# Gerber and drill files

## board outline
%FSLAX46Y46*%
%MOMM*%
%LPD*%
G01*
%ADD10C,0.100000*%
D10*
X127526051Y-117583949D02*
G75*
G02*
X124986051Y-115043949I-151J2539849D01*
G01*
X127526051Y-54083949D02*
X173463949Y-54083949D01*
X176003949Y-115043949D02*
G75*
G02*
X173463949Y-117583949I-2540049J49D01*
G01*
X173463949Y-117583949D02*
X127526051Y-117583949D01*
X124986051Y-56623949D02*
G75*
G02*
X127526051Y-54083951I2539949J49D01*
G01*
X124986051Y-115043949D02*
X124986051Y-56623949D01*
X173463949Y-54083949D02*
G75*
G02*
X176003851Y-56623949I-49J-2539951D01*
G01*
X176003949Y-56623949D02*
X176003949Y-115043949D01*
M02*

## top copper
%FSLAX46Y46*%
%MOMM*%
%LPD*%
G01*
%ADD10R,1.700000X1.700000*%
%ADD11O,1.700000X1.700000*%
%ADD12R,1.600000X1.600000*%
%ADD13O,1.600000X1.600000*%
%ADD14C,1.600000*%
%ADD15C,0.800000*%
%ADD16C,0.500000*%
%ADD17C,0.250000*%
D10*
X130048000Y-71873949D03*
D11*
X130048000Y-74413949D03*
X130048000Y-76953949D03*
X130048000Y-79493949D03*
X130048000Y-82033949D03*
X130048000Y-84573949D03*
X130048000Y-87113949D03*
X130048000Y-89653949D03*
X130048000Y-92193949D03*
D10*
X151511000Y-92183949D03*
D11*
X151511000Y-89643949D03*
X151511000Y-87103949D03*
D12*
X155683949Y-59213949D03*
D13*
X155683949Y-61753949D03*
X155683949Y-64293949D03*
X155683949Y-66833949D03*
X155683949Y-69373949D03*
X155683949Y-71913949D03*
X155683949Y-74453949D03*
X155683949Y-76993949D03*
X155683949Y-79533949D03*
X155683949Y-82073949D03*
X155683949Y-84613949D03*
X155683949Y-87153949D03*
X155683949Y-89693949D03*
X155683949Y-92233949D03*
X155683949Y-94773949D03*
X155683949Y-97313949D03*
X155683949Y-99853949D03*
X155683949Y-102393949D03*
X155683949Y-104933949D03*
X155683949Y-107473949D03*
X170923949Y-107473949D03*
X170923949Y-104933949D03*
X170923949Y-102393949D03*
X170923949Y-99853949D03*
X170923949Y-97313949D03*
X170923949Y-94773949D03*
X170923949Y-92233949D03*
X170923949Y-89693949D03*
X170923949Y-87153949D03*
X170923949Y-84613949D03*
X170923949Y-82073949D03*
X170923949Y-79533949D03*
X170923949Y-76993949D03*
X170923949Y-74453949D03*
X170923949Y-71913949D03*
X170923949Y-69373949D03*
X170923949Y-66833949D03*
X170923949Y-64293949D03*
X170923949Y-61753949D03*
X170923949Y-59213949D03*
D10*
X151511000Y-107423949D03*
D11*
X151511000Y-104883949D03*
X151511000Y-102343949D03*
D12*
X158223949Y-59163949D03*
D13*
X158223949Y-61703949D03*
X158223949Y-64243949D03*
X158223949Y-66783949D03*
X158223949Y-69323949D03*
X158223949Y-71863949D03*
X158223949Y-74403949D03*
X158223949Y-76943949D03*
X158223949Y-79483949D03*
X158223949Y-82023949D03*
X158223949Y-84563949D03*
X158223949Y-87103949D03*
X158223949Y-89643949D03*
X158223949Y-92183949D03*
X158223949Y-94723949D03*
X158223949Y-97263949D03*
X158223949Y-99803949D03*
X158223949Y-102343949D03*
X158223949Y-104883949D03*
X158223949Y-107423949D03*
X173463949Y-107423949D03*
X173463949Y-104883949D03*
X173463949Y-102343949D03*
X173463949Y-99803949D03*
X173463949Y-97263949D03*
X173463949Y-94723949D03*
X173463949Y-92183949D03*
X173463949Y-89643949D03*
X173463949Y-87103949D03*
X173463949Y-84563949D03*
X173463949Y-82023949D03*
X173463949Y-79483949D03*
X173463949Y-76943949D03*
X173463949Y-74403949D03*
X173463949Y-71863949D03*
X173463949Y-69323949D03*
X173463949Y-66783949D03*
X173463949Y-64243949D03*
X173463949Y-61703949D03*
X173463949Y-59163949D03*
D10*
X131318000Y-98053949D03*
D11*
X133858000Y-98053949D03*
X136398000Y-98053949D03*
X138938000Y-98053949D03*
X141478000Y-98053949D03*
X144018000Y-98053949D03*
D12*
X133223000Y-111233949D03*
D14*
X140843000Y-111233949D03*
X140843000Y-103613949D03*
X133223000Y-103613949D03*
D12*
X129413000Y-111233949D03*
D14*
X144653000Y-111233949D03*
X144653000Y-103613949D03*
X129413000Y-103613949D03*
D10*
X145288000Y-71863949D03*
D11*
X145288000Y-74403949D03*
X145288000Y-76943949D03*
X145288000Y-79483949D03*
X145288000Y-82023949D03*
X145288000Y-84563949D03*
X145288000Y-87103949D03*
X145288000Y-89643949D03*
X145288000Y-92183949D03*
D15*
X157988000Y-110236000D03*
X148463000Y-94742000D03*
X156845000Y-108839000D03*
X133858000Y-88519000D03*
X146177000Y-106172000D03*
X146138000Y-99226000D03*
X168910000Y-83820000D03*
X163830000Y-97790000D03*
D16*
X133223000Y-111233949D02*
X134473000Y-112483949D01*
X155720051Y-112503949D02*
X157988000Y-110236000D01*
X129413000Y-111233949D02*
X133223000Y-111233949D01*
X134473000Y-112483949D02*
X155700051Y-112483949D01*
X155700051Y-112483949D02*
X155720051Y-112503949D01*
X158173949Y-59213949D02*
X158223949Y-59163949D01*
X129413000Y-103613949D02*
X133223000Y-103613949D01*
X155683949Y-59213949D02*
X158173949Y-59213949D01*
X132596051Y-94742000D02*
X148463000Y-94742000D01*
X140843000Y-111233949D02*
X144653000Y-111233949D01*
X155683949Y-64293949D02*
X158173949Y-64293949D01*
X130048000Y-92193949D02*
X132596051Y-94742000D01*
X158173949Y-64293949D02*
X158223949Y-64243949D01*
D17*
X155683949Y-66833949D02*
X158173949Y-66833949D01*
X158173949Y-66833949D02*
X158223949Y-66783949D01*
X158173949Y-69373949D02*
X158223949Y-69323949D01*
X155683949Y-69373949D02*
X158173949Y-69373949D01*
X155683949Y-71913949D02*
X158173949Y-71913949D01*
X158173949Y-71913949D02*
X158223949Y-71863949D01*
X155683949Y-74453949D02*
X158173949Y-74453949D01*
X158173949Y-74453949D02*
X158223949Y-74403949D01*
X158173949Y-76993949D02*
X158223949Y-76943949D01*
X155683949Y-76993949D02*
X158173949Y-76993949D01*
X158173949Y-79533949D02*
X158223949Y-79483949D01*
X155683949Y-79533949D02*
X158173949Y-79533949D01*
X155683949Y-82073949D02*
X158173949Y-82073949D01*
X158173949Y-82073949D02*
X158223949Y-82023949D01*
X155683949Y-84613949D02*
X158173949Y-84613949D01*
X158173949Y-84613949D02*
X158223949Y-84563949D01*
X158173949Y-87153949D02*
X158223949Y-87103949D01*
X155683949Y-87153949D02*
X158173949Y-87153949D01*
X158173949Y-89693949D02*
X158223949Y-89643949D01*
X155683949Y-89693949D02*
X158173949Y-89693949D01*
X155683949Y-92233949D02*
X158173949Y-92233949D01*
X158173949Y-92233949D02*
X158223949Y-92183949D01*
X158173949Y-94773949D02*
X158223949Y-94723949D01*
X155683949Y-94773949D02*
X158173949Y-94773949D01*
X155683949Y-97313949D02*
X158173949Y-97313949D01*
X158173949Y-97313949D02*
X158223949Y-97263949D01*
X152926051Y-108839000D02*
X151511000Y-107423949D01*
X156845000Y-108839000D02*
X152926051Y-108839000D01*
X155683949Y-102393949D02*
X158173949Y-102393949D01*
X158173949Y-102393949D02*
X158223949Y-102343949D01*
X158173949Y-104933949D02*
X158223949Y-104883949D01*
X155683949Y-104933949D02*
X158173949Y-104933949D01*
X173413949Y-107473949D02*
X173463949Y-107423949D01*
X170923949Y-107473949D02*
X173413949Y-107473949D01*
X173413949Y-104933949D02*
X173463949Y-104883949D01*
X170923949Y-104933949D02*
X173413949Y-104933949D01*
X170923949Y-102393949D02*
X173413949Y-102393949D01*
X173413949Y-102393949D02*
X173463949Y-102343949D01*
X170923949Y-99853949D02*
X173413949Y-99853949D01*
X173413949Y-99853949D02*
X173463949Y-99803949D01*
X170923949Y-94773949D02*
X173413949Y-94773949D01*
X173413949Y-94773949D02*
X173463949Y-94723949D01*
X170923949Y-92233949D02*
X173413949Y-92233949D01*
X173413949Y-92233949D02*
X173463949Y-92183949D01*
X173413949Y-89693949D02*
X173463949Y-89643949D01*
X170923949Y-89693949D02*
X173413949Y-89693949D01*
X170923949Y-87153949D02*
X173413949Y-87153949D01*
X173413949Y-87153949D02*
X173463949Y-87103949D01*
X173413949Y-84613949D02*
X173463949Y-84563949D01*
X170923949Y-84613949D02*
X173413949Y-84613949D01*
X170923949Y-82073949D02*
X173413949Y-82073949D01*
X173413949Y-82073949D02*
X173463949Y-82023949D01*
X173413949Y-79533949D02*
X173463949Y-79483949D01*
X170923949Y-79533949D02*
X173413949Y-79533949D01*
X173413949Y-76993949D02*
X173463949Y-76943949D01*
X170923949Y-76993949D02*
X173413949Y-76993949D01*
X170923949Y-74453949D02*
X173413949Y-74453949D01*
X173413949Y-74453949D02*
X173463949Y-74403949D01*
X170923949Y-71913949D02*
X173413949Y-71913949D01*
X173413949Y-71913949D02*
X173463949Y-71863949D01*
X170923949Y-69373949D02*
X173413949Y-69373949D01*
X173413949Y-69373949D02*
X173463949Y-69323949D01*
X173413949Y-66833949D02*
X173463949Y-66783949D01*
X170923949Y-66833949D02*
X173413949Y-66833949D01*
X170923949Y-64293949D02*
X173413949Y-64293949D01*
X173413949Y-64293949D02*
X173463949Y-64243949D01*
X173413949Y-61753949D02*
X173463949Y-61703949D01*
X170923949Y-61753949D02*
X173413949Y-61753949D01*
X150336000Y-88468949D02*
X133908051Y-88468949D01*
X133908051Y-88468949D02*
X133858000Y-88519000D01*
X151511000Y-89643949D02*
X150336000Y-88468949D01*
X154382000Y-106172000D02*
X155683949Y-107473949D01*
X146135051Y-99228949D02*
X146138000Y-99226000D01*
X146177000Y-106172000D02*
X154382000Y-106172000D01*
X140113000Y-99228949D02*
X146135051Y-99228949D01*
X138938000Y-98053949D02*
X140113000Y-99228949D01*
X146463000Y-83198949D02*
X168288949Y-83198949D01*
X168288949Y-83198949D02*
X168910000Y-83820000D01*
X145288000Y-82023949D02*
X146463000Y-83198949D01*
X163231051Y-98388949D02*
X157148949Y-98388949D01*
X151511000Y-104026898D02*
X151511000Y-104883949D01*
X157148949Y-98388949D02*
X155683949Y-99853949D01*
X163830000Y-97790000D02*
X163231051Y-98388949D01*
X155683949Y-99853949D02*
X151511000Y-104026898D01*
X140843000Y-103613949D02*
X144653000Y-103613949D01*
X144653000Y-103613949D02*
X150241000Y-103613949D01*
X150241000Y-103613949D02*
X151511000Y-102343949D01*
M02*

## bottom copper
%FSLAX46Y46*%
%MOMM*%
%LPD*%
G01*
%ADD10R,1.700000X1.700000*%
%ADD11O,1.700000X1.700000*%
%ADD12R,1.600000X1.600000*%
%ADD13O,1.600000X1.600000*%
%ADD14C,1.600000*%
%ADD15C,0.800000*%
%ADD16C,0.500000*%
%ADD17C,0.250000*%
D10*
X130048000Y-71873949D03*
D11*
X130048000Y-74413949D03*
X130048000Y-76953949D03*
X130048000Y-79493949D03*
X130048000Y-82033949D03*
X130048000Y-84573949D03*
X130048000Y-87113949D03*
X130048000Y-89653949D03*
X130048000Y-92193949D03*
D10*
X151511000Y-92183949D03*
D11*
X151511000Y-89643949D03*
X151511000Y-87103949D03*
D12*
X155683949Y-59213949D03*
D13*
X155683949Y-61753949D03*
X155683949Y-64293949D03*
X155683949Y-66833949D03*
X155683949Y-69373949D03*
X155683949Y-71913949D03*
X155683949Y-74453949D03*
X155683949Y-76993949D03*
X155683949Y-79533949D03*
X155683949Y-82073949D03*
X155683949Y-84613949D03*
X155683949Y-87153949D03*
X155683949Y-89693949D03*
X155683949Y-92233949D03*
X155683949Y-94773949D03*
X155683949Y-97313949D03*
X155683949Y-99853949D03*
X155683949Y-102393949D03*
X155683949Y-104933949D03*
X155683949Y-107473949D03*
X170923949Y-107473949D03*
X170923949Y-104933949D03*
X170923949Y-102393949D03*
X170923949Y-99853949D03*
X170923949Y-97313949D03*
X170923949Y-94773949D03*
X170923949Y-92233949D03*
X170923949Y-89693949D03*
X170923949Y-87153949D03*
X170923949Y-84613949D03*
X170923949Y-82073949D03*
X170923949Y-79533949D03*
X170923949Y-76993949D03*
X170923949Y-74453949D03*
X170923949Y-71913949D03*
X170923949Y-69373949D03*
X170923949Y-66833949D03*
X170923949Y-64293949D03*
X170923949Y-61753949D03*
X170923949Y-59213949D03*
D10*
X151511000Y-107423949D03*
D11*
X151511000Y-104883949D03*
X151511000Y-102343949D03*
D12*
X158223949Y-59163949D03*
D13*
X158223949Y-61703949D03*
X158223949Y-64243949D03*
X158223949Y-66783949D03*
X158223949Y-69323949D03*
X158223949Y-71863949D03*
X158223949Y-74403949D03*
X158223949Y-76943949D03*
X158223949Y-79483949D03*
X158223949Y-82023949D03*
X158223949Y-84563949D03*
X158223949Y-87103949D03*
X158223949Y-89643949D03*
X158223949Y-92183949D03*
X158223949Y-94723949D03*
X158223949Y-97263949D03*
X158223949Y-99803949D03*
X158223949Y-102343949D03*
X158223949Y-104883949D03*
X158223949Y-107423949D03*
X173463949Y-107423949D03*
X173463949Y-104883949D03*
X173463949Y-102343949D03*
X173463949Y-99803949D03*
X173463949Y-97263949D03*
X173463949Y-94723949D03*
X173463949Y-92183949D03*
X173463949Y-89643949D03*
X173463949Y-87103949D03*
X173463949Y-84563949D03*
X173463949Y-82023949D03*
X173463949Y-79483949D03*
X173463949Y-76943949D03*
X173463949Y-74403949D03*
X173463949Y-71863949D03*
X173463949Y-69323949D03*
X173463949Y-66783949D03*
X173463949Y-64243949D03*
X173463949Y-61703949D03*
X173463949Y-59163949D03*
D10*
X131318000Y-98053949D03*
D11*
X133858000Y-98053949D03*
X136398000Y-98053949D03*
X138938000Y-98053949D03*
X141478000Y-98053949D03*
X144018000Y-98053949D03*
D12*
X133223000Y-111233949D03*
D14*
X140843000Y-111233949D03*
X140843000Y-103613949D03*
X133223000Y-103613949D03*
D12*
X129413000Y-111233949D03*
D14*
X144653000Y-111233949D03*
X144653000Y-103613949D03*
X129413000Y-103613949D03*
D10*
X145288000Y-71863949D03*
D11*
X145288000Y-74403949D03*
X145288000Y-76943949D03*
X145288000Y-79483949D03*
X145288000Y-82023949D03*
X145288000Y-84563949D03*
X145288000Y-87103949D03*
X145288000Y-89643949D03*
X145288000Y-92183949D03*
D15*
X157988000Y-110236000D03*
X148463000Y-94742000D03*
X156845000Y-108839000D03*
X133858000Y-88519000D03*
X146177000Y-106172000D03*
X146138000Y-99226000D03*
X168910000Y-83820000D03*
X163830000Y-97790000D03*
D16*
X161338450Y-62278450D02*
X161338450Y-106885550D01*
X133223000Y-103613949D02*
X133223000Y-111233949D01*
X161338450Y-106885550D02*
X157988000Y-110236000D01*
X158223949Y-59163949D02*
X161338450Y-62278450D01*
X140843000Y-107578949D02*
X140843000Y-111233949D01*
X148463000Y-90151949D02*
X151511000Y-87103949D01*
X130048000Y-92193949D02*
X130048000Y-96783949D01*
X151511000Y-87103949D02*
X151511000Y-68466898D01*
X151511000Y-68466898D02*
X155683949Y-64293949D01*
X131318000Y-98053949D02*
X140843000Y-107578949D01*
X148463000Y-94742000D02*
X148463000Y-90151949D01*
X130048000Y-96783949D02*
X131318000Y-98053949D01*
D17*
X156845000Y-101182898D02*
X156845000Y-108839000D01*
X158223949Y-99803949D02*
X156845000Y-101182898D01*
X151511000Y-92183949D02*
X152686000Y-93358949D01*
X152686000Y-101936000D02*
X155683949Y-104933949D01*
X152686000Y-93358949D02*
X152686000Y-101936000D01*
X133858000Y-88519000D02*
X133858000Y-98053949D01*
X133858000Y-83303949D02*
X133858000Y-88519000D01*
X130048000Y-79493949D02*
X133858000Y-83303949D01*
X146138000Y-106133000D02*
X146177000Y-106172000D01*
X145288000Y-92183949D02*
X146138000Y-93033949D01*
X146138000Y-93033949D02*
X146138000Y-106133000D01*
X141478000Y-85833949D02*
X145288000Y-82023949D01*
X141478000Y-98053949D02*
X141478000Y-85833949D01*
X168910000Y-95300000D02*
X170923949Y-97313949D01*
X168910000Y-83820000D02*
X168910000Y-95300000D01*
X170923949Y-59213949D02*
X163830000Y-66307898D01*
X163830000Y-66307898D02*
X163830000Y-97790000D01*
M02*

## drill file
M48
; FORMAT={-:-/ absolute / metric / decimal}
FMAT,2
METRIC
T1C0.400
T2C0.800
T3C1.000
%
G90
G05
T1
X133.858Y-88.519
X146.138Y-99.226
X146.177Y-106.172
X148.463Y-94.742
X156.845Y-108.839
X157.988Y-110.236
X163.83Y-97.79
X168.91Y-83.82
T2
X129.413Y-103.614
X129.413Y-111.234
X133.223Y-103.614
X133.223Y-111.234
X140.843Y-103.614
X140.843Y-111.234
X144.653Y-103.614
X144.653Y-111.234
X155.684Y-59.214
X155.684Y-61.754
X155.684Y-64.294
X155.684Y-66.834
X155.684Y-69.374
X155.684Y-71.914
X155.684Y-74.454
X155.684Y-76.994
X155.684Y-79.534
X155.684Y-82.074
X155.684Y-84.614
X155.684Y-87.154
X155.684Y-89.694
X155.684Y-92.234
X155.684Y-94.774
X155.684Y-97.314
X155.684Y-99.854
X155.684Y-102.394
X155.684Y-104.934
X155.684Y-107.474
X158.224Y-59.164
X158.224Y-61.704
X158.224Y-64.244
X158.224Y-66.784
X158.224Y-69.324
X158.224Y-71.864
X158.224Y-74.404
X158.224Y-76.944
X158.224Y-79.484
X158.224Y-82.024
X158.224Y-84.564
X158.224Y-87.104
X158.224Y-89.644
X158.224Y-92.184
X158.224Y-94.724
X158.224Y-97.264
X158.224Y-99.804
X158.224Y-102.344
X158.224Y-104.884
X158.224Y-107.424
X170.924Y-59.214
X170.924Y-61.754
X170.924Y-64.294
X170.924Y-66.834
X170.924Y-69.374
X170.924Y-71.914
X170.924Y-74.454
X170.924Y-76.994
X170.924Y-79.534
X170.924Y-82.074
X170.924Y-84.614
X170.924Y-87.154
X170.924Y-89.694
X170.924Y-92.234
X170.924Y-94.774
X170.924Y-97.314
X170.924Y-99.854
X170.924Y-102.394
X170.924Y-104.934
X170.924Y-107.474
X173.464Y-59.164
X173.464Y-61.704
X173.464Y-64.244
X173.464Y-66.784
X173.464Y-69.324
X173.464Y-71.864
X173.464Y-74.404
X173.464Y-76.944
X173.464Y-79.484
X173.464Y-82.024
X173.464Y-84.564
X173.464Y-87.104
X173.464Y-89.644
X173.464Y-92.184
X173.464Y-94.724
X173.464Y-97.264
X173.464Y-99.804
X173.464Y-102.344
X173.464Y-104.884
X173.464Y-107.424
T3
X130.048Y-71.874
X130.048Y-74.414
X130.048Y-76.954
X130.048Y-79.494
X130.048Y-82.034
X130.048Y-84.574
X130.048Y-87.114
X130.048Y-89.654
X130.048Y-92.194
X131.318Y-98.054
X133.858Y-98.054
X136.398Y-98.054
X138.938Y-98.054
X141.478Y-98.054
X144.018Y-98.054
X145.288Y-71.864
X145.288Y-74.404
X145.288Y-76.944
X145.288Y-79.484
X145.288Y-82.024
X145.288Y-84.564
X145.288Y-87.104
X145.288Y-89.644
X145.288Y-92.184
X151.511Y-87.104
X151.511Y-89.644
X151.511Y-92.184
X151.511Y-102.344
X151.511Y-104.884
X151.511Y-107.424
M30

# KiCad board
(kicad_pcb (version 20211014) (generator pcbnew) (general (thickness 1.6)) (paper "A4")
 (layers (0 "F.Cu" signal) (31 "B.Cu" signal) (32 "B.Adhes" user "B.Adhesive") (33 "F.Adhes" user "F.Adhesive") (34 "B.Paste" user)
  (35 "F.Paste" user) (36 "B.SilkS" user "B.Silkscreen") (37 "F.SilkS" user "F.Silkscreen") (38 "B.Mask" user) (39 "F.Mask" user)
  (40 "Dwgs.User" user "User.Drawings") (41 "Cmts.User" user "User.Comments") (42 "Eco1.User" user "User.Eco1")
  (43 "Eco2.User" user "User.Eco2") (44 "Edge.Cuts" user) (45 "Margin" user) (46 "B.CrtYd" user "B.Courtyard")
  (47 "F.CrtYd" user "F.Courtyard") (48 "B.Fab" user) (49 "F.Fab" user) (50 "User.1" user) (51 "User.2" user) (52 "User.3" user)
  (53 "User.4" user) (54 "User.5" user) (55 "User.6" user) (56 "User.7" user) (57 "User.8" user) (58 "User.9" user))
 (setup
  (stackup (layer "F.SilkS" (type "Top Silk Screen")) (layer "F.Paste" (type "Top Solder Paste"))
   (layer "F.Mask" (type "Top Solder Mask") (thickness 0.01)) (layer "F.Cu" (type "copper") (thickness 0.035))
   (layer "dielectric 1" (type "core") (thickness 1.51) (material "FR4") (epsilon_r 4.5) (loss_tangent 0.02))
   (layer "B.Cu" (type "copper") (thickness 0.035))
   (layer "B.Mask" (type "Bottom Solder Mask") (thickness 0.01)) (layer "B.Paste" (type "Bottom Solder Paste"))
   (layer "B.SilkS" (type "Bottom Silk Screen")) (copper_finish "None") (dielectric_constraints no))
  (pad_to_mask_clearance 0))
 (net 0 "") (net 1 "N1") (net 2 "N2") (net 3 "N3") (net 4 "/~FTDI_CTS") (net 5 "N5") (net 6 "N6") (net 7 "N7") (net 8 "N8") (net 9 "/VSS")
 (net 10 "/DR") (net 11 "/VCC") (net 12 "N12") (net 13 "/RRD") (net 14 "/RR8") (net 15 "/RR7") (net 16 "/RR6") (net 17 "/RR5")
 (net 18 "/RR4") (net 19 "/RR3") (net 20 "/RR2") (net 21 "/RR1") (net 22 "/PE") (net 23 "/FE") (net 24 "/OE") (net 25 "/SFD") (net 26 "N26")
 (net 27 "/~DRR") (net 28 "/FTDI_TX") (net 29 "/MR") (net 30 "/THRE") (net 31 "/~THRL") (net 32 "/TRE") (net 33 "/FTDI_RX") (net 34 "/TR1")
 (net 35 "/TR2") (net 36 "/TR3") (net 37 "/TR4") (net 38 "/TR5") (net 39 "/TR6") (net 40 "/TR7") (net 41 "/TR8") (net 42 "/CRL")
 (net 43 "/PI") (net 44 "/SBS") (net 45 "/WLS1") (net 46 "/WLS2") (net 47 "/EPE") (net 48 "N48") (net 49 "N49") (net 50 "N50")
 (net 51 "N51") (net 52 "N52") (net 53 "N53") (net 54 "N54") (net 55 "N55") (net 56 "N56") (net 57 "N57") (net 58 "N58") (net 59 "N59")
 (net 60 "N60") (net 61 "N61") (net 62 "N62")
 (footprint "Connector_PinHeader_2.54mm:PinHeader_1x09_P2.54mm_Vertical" (layer "F.Cu") (at 130.048 71.873949)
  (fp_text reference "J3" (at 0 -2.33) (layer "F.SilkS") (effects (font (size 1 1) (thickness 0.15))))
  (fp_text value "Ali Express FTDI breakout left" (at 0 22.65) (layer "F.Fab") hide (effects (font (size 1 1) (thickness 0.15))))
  (pad "1" thru_hole rect (at 0 0) (size 1.7 1.7) (drill 1) (layers *.Cu *.Mask) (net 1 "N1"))
  (pad "2" thru_hole oval (at 0 2.54) (size 1.7 1.7) (drill 1) (layers *.Cu *.Mask) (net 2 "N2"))
  (pad "3" thru_hole oval (at 0 5.08) (size 1.7 1.7) (drill 1) (layers *.Cu *.Mask) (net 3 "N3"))
  (pad "4" thru_hole oval (at 0 7.62) (size 1.7 1.7) (drill 1) (layers *.Cu *.Mask) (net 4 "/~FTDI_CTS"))
  (pad "5" thru_hole oval (at 0 10.16) (size 1.7 1.7) (drill 1) (layers *.Cu *.Mask) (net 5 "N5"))
  (pad "6" thru_hole oval (at 0 12.7) (size 1.7 1.7) (drill 1) (layers *.Cu *.Mask) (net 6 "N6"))
  (pad "7" thru_hole oval (at 0 15.24) (size 1.7 1.7) (drill 1) (layers *.Cu *.Mask) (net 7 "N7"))
  (pad "8" thru_hole oval (at 0 17.78) (size 1.7 1.7) (drill 1) (layers *.Cu *.Mask) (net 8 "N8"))
  (pad "9" thru_hole oval (at 0 20.32) (size 1.7 1.7) (drill 1) (layers *.Cu *.Mask) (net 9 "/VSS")))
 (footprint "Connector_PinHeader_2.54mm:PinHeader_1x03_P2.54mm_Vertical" (layer "F.Cu") (at 151.511 92.183949 180)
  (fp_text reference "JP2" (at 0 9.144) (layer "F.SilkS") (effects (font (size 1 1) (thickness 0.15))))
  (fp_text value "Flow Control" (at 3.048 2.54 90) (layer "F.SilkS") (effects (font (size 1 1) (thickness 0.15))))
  (pad "1" thru_hole rect (at 0 0 180) (size 1.7 1.7) (drill 1) (layers *.Cu *.Mask) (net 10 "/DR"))
  (pad "2" thru_hole oval (at 0 2.54 180) (size 1.7 1.7) (drill 1) (layers *.Cu *.Mask) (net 4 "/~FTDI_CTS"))
  (pad "3" thru_hole oval (at 0 5.08 180) (size 1.7 1.7) (drill 1) (layers *.Cu *.Mask) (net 9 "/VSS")))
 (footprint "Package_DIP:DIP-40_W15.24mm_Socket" (layer "F.Cu") (at 155.683949 59.213949)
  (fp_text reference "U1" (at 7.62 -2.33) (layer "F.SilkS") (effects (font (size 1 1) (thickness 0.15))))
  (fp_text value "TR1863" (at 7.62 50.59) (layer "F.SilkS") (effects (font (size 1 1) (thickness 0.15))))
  (pad "1" thru_hole rect (at 0 0) (size 1.6 1.6) (drill 0.8) (layers *.Cu *.Mask) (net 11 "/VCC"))
  (pad "2" thru_hole oval (at 0 2.54) (size 1.6 1.6) (drill 0.8) (layers *.Cu *.Mask) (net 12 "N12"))
  (pad "3" thru_hole oval (at 0 5.08) (size 1.6 1.6) (drill 0.8) (layers *.Cu *.Mask) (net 9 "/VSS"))
  (pad "4" thru_hole oval (at 0 7.62) (size 1.6 1.6) (drill 0.8) (layers *.Cu *.Mask) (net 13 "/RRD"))
  (pad "5" thru_hole oval (at 0 10.16) (size 1.6 1.6) (drill 0.8) (layers *.Cu *.Mask) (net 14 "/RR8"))
  (pad "6" thru_hole oval (at 0 12.7) (size 1.6 1.6) (drill 0.8) (layers *.Cu *.Mask) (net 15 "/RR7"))
  (pad "7" thru_hole oval (at 0 15.24) (size 1.6 1.6) (drill 0.8) (layers *.Cu *.Mask) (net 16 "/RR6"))
  (pad "8" thru_hole oval (at 0 17.78) (size 1.6 1.6) (drill 0.8) (layers *.Cu *.Mask) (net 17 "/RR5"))
  (pad "9" thru_hole oval (at 0 20.32) (size 1.6 1.6) (drill 0.8) (layers *.Cu *.Mask) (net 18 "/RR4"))
  (pad "10" thru_hole oval (at 0 22.86) (size 1.6 1.6) (drill 0.8) (layers *.Cu *.Mask) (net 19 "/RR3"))
  (pad "11" thru_hole oval (at 0 25.4) (size 1.6 1.6) (drill 0.8) (layers *.Cu *.Mask) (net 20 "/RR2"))
  (pad "12" thru_hole oval (at 0 27.94) (size 1.6 1.6) (drill 0.8) (layers *.Cu *.Mask) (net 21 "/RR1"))
  (pad "13" thru_hole oval (at 0 30.48) (size 1.6 1.6) (drill 0.8) (layers *.Cu *.Mask) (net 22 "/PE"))
  (pad "14" thru_hole oval (at 0 33.02) (size 1.6 1.6) (drill 0.8) (layers *.Cu *.Mask) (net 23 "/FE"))
  (pad "15" thru_hole oval (at 0 35.56) (size 1.6 1.6) (drill 0.8) (layers *.Cu *.Mask) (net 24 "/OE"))
  (pad "16" thru_hole oval (at 0 38.1) (size 1.6 1.6) (drill 0.8) (layers *.Cu *.Mask) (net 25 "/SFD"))
  (pad "17" thru_hole oval (at 0 40.64) (size 1.6 1.6) (drill 0.8) (layers *.Cu *.Mask) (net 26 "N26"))
  (pad "18" thru_hole oval (at 0 43.18) (size 1.6 1.6) (drill 0.8) (layers *.Cu *.Mask) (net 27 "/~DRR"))
  (pad "19" thru_hole oval (at 0 45.72) (size 1.6 1.6) (drill 0.8) (layers *.Cu *.Mask) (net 10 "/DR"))
  (pad "20" thru_hole oval (at 0 48.26) (size 1.6 1.6) (drill 0.8) (layers *.Cu *.Mask) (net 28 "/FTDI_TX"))
  (pad "21" thru_hole oval (at 15.24 48.26) (size 1.6 1.6) (drill 0.8) (layers *.Cu *.Mask) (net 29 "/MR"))
  (pad "22" thru_hole oval (at 15.24 45.72) (size 1.6 1.6) (drill 0.8) (layers *.Cu *.Mask) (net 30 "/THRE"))
  (pad "23" thru_hole oval (at 15.24 43.18) (size 1.6 1.6) (drill 0.8) (layers *.Cu *.Mask) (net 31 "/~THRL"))
  (pad "24" thru_hole oval (at 15.24 40.64) (size 1.6 1.6) (drill 0.8) (layers *.Cu *.Mask) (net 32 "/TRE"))
  (pad "25" thru_hole oval (at 15.24 38.1) (size 1.6 1.6) (drill 0.8) (layers *.Cu *.Mask) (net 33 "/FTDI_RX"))
  (pad "26" thru_hole oval (at 15.24 35.56) (size 1.6 1.6) (drill 0.8) (layers *.Cu *.Mask) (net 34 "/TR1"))
  (pad "27" thru_hole oval (at 15.24 33.02) (size 1.6 1.6) (drill 0.8) (layers *.Cu *.Mask) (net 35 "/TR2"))
  (pad "28" thru_hole oval (at 15.24 30.48) (size 1.6 1.6) (drill 0.8) (layers *.Cu *.Mask) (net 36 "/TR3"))
  (pad "29" thru_hole oval (at 15.24 27.94) (size 1.6 1.6) (drill 0.8) (layers *.Cu *.Mask) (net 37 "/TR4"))
  (pad "30" thru_hole oval (at 15.24 25.4) (size 1.6 1.6) (drill 0.8) (layers *.Cu *.Mask) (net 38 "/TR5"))
  (pad "31" thru_hole oval (at 15.24 22.86) (size 1.6 1.6) (drill 0.8) (layers *.Cu *.Mask) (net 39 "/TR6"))
  (pad "32" thru_hole oval (at 15.24 20.32) (size 1.6 1.6) (drill 0.8) (layers *.Cu *.Mask) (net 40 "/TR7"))
  (pad "33" thru_hole oval (at 15.24 17.78) (size 1.6 1.6) (drill 0.8) (layers *.Cu *.Mask) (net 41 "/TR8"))
  (pad "34" thru_hole oval (at 15.24 15.24) (size 1.6 1.6) (drill 0.8) (layers *.Cu *.Mask) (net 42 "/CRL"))
  (pad "35" thru_hole oval (at 15.24 12.7) (size 1.6 1.6) (drill 0.8) (layers *.Cu *.Mask) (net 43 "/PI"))
  (pad "36" thru_hole oval (at 15.24 10.16) (size 1.6 1.6) (drill 0.8) (layers *.Cu *.Mask) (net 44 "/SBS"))
  (pad "37" thru_hole oval (at 15.24 7.62) (size 1.6 1.6) (drill 0.8) (layers *.Cu *.Mask) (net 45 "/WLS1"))
  (pad "38" thru_hole oval (at 15.24 5.08) (size 1.6 1.6) (drill 0.8) (layers *.Cu *.Mask) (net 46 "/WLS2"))
  (pad "39" thru_hole oval (at 15.24 2.54) (size 1.6 1.6) (drill 0.8) (layers *.Cu *.Mask) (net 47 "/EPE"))
  (pad "40" thru_hole oval (at 15.24 0) (size 1.6 1.6) (drill 0.8) (layers *.Cu *.Mask) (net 26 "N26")))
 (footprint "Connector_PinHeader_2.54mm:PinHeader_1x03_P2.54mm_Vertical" (layer "F.Cu") (at 151.511 107.423949 180)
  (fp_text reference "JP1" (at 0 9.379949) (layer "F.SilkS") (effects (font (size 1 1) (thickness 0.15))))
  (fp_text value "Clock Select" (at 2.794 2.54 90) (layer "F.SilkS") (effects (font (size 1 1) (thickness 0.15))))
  (pad "1" thru_hole rect (at 0 0 180) (size 1.7 1.7) (drill 1) (layers *.Cu *.Mask) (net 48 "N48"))
  (pad "2" thru_hole oval (at 0 2.54 180) (size 1.7 1.7) (drill 1) (layers *.Cu *.Mask) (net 26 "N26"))
  (pad "3" thru_hole oval (at 0 5.08 180) (size 1.7 1.7) (drill 1) (layers *.Cu *.Mask) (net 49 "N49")))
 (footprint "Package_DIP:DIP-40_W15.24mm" (layer "F.Cu") (at 158.223949 59.163949)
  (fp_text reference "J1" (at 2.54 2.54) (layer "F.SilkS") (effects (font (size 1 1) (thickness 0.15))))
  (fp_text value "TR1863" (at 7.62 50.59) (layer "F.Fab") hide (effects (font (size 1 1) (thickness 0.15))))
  (pad "1" thru_hole rect (at 0 0) (size 1.6 1.6) (drill 0.8) (layers *.Cu *.Mask) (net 11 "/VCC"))
  (pad "2" thru_hole oval (at 0 2.54) (size 1.6 1.6) (drill 0.8) (layers *.Cu *.Mask) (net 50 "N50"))
  (pad "3" thru_hole oval (at 0 5.08) (size 1.6 1.6) (drill 0.8) (layers *.Cu *.Mask) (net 9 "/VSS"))
  (pad "4" thru_hole oval (at 0 7.62) (size 1.6 1.6) (drill 0.8) (layers *.Cu *.Mask) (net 13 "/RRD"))
  (pad "5" thru_hole oval (at 0 10.16) (size 1.6 1.6) (drill 0.8) (layers *.Cu *.Mask) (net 14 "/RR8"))
  (pad "6" thru_hole oval (at 0 12.7) (size 1.6 1.6) (drill 0.8) (layers *.Cu *.Mask) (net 15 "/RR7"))
  (pad "7" thru_hole oval (at 0 15.24) (size 1.6 1.6) (drill 0.8) (layers *.Cu *.Mask) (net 16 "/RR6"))
  (pad "8" thru_hole oval (at 0 17.78) (size 1.6 1.6) (drill 0.8) (layers *.Cu *.Mask) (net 17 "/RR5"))
  (pad "9" thru_hole oval (at 0 20.32) (size 1.6 1.6) (drill 0.8) (layers *.Cu *.Mask) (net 18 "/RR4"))
  (pad "10" thru_hole oval (at 0 22.86) (size 1.6 1.6) (drill 0.8) (layers *.Cu *.Mask) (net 19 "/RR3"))
  (pad "11" thru_hole oval (at 0 25.4) (size 1.6 1.6) (drill 0.8) (layers *.Cu *.Mask) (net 20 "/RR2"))
  (pad "12" thru_hole oval (at 0 27.94) (size 1.6 1.6) (drill 0.8) (layers *.Cu *.Mask) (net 21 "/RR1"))
  (pad "13" thru_hole oval (at 0 30.48) (size 1.6 1.6) (drill 0.8) (layers *.Cu *.Mask) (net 22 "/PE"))
  (pad "14" thru_hole oval (at 0 33.02) (size 1.6 1.6) (drill 0.8) (layers *.Cu *.Mask) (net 23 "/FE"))
  (pad "15" thru_hole oval (at 0 35.56) (size 1.6 1.6) (drill 0.8) (layers *.Cu *.Mask) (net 24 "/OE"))
  (pad "16" thru_hole oval (at 0 38.1) (size 1.6 1.6) (drill 0.8) (layers *.Cu *.Mask) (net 25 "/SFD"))
  (pad "17" thru_hole oval (at 0 40.64) (size 1.6 1.6) (drill 0.8) (layers *.Cu *.Mask) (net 48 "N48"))
  (pad "18" thru_hole oval (at 0 43.18) (size 1.6 1.6) (drill 0.8) (layers *.Cu *.Mask) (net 27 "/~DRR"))
  (pad "19" thru_hole oval (at 0 45.72) (size 1.6 1.6) (drill 0.8) (layers *.Cu *.Mask) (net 10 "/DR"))
  (pad "20" thru_hole oval (at 0 48.26) (size 1.6 1.6) (drill 0.8) (layers *.Cu *.Mask) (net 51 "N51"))
  (pad "21" thru_hole oval (at 15.24 48.26) (size 1.6 1.6) (drill 0.8) (layers *.Cu *.Mask) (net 29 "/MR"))
  (pad "22" thru_hole oval (at 15.24 45.72) (size 1.6 1.6) (drill 0.8) (layers *.Cu *.Mask) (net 30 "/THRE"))
  (pad "23" thru_hole oval (at 15.24 43.18) (size 1.6 1.6) (drill 0.8) (layers *.Cu *.Mask) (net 31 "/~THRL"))
  (pad "24" thru_hole oval (at 15.24 40.64) (size 1.6 1.6) (drill 0.8) (layers *.Cu *.Mask) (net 32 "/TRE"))
  (pad "25" thru_hole oval (at 15.24 38.1) (size 1.6 1.6) (drill 0.8) (layers *.Cu *.Mask) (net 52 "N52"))
  (pad "26" thru_hole oval (at 15.24 35.56) (size 1.6 1.6) (drill 0.8) (layers *.Cu *.Mask) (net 34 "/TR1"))
  (pad "27" thru_hole oval (at 15.24 33.02) (size 1.6 1.6) (drill 0.8) (layers *.Cu *.Mask) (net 35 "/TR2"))
  (pad "28" thru_hole oval (at 15.24 30.48) (size 1.6 1.6) (drill 0.8) (layers *.Cu *.Mask) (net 36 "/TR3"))
  (pad "29" thru_hole oval (at 15.24 27.94) (size 1.6 1.6) (drill 0.8) (layers *.Cu *.Mask) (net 37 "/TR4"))
  (pad "30" thru_hole oval (at 15.24 25.4) (size 1.6 1.6) (drill 0.8) (layers *.Cu *.Mask) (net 38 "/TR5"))
  (pad "31" thru_hole oval (at 15.24 22.86) (size 1.6 1.6) (drill 0.8) (layers *.Cu *.Mask) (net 39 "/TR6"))
  (pad "32" thru_hole oval (at 15.24 20.32) (size 1.6 1.6) (drill 0.8) (layers *.Cu *.Mask) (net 40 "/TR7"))
  (pad "33" thru_hole oval (at 15.24 17.78) (size 1.6 1.6) (drill 0.8) (layers *.Cu *.Mask) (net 41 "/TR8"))
  (pad "34" thru_hole oval (at 15.24 15.24) (size 1.6 1.6) (drill 0.8) (layers *.Cu *.Mask) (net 42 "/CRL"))
  (pad "35" thru_hole oval (at 15.24 12.7) (size 1.6 1.6) (drill 0.8) (layers *.Cu *.Mask) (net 43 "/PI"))
  (pad "36" thru_hole oval (at 15.24 10.16) (size 1.6 1.6) (drill 0.8) (layers *.Cu *.Mask) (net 44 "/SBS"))
  (pad "37" thru_hole oval (at 15.24 7.62) (size 1.6 1.6) (drill 0.8) (layers *.Cu *.Mask) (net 45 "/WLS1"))
  (pad "38" thru_hole oval (at 15.24 5.08) (size 1.6 1.6) (drill 0.8) (layers *.Cu *.Mask) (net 46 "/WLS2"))
  (pad "39" thru_hole oval (at 15.24 2.54) (size 1.6 1.6) (drill 0.8) (layers *.Cu *.Mask) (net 47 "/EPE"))
  (pad "40" thru_hole oval (at 15.24 0) (size 1.6 1.6) (drill 0.8) (layers *.Cu *.Mask) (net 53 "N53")))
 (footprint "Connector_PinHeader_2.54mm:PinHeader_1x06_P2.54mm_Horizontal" (layer "F.Cu") (at 131.318 98.053949 90)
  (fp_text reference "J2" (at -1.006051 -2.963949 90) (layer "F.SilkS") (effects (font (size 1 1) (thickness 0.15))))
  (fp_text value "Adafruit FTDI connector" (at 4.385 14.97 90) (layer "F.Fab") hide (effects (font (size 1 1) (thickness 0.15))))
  (pad "1" thru_hole rect (at 0 0 90) (size 1.7 1.7) (drill 1) (layers *.Cu *.Mask) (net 9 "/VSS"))
  (pad "2" thru_hole oval (at 0 2.54 90) (size 1.7 1.7) (drill 1) (layers *.Cu *.Mask) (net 4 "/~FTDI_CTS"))
  (pad "3" thru_hole oval (at 0 5.08 90) (size 1.7 1.7) (drill 1) (layers *.Cu *.Mask) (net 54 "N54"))
  (pad "4" thru_hole oval (at 0 7.62 90) (size 1.7 1.7) (drill 1) (layers *.Cu *.Mask) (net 28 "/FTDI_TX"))
  (pad "5" thru_hole oval (at 0 10.16 90) (size 1.7 1.7) (drill 1) (layers *.Cu *.Mask) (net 33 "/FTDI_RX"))
  (pad "6" thru_hole oval (at 0 12.7 90) (size 1.7 1.7) (drill 1) (layers *.Cu *.Mask) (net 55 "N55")))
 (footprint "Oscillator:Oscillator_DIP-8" (layer "F.Cu") (at 133.223 111.233949)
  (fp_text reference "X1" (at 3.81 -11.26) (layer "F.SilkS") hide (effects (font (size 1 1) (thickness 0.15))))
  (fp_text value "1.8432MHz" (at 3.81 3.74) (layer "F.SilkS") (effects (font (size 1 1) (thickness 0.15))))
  (pad "1" thru_hole rect (at 0 0) (size 1.6 1.6) (drill 0.8) (layers *.Cu *.Mask) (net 11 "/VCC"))
  (pad "4" thru_hole circle (at 7.62 0) (size 1.6 1.6) (drill 0.8) (layers *.Cu *.Mask) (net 9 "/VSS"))
  (pad "5" thru_hole circle (at 7.62 -7.62) (size 1.6 1.6) (drill 0.8) (layers *.Cu *.Mask) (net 49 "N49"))
  (pad "8" thru_hole circle (at 0 -7.62) (size 1.6 1.6) (drill 0.8) (layers *.Cu *.Mask) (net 11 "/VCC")))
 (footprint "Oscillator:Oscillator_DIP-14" (layer "F.Cu") (at 129.413 111.233949)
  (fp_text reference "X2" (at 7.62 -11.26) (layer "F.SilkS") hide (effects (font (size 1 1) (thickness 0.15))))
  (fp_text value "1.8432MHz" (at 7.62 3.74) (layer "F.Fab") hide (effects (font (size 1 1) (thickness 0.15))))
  (pad "1" thru_hole rect (at 0 0) (size 1.6 1.6) (drill 0.8) (layers *.Cu *.Mask) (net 11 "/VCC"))
  (pad "7" thru_hole circle (at 15.24 0) (size 1.6 1.6) (drill 0.8) (layers *.Cu *.Mask) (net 9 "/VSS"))
  (pad "8" thru_hole circle (at 15.24 -7.62) (size 1.6 1.6) (drill 0.8) (layers *.Cu *.Mask) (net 49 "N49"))
  (pad "14" thru_hole circle (at 0 -7.62) (size 1.6 1.6) (drill 0.8) (layers *.Cu *.Mask) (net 11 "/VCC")))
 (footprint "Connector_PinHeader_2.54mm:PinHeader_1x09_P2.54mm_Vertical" (layer "F.Cu") (at 145.288 71.863949)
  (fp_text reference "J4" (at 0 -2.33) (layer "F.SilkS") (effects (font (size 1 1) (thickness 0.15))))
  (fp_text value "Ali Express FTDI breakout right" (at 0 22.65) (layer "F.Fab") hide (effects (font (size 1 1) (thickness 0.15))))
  (pad "1" thru_hole rect (at 0 0) (size 1.7 1.7) (drill 1) (layers *.Cu *.Mask) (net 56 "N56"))
  (pad "2" thru_hole oval (at 0 2.54) (size 1.7 1.7) (drill 1) (layers *.Cu *.Mask) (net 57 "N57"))
  (pad "3" thru_hole oval (at 0 5.08) (size 1.7 1.7) (drill 1) (layers *.Cu *.Mask) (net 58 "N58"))
  (pad "4" thru_hole oval (at 0 7.62) (size 1.7 1.7) (drill 1) (layers *.Cu *.Mask) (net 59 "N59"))
  (pad "5" thru_hole oval (at 0 10.16) (size 1.7 1.7) (drill 1) (layers *.Cu *.Mask) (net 33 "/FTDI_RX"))
  (pad "6" thru_hole oval (at 0 12.7) (size 1.7 1.7) (drill 1) (layers *.Cu *.Mask) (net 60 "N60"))
  (pad "7" thru_hole oval (at 0 15.24) (size 1.7 1.7) (drill 1) (layers *.Cu *.Mask) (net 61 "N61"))
  (pad "8" thru_hole oval (at 0 17.78) (size 1.7 1.7) (drill 1) (layers *.Cu *.Mask) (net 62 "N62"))
  (pad "9" thru_hole oval (at 0 20.32) (size 1.7 1.7) (drill 1) (layers *.Cu *.Mask) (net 28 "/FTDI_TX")))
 (gr_arc (start 127.526051 117.583949) (mid 125.729951 116.840021) (end 124.986051 115.043949) (layer "Edge.Cuts") (width 0.1))
 (gr_line (start 127.526051 54.083949) (end 173.463949 54.083949) (layer "Edge.Cuts") (width 0.1))
 (gr_arc (start 176.003949 115.043949) (mid 175.26 116.84) (end 173.463949 117.583949) (layer "Edge.Cuts") (width 0.1))
 (gr_line (start 173.463949 117.583949) (end 127.526051 117.583949) (layer "Edge.Cuts") (width 0.1))
 (gr_arc (start 124.986051 56.623949) (mid 125.729985 54.827883) (end 127.526051 54.083949) (layer "Edge.Cuts") (width 0.1))
 (gr_line (start 124.986051 115.043949) (end 124.986051 56.623949) (layer "Edge.Cuts") (width 0.1))
 (gr_arc (start 173.463949 54.083949) (mid 175.26 54.827898) (end 176.003949 56.623949) (layer "Edge.Cuts") (width 0.1))
 (gr_line (start 176.003949 56.623949) (end 176.003949 115.043949) (layer "Edge.Cuts") (width 0.1))
 (segment (start 133.223 111.233949) (end 134.473 112.483949) (width 0.5) (layer "F.Cu") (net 11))
 (segment (start 155.720051 112.503949) (end 157.988 110.236) (width 0.5) (layer "F.Cu") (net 11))
 (segment (start 129.413 111.233949) (end 133.223 111.233949) (width 0.5) (layer "F.Cu") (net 11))
 (segment (start 134.473 112.483949) (end 155.700051 112.483949) (width 0.5) (layer "F.Cu") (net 11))
 (segment (start 155.700051 112.483949) (end 155.720051 112.503949) (width 0.5) (layer "F.Cu") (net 11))
 (segment (start 158.173949 59.213949) (end 158.223949 59.163949) (width 0.5) (layer "F.Cu") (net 11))
 (segment (start 129.413 103.613949) (end 133.223 103.613949) (width 0.5) (layer "F.Cu") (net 11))
 (segment (start 155.683949 59.213949) (end 158.173949 59.213949) (width 0.5) (layer "F.Cu") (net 11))
 (via (at 157.988 110.236) (size 0.8) (drill 0.4) (layers "F.Cu" "B.Cu") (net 11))
 (segment (start 161.33845 62.27845) (end 161.33845 106.88555) (width 0.5) (layer "B.Cu") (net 11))
 (segment (start 133.223 103.613949) (end 133.223 111.233949) (width 0.5) (layer "B.Cu") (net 11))
 (segment (start 161.33845 106.88555) (end 157.988 110.236) (width 0.5) (layer "B.Cu") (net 11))
 (segment (start 158.223949 59.163949) (end 161.33845 62.27845) (width 0.5) (layer "B.Cu") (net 11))
 (segment (start 132.596051 94.742) (end 148.463 94.742) (width 0.5) (layer "F.Cu") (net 9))
 (segment (start 140.843 111.233949) (end 144.653 111.233949) (width 0.5) (layer "F.Cu") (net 9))
 (segment (start 155.683949 64.293949) (end 158.173949 64.293949) (width 0.5) (layer "F.Cu") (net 9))
 (segment (start 130.048 92.193949) (end 132.596051 94.742) (width 0.5) (layer "F.Cu") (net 9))
 (segment (start 158.173949 64.293949) (end 158.223949 64.243949) (width 0.5) (layer "F.Cu") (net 9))
 (via (at 148.463 94.742) (size 0.8) (drill 0.4) (layers "F.Cu" "B.Cu") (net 9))
 (segment (start 140.843 107.578949) (end 140.843 111.233949) (width 0.5) (layer "B.Cu") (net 9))
 (segment (start 148.463 90.151949) (end 151.511 87.103949) (width 0.5) (layer "B.Cu") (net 9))
 (segment (start 130.048 92.193949) (end 130.048 96.783949) (width 0.5) (layer "B.Cu") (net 9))
 (segment (start 151.511 87.103949) (end 151.511 68.466898) (width 0.5) (layer "B.Cu") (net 9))
 (segment (start 151.511 68.466898) (end 155.683949 64.293949) (width 0.5) (layer "B.Cu") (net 9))
 (segment (start 131.318 98.053949) (end 140.843 107.578949) (width 0.5) (layer "B.Cu") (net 9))
 (segment (start 148.463 94.742) (end 148.463 90.151949) (width 0.5) (layer "B.Cu") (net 9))
 (segment (start 130.048 96.783949) (end 131.318 98.053949) (width 0.5) (layer "B.Cu") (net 9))
 (segment (start 155.683949 66.833949) (end 158.173949 66.833949) (width 0.25) (layer "F.Cu") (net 13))
 (segment (start 158.173949 66.833949) (end 158.223949 66.783949) (width 0.25) (layer "F.Cu") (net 13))
 (segment (start 158.173949 69.373949) (end 158.223949 69.323949) (width 0.25) (layer "F.Cu") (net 14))
 (segment (start 155.683949 69.373949) (end 158.173949 69.373949) (width 0.25) (layer "F.Cu") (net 14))
 (segment (start 155.683949 71.913949) (end 158.173949 71.913949) (width 0.25) (layer "F.Cu") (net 15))
 (segment (start 158.173949 71.913949) (end 158.223949 71.863949) (width 0.25) (layer "F.Cu") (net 15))
 (segment (start 155.683949 74.453949) (end 158.173949 74.453949) (width 0.25) (layer "F.Cu") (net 16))
 (segment (start 158.173949 74.453949) (end 158.223949 74.403949) (width 0.25) (layer "F.Cu") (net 16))
 (segment (start 158.173949 76.993949) (end 158.223949 76.943949) (width 0.25) (layer "F.Cu") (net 17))
 (segment (start 155.683949 76.993949) (end 158.173949 76.993949) (width 0.25) (layer "F.Cu") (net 17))
 (segment (start 158.173949 79.533949) (end 158.223949 79.483949) (width 0.25) (layer "F.Cu") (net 18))
 (segment (start 155.683949 79.533949) (end 158.173949 79.533949) (width 0.25) (layer "F.Cu") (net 18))
 (segment (start 155.683949 82.073949) (end 158.173949 82.073949) (width 0.25) (layer "F.Cu") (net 19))
 (segment (start 158.173949 82.073949) (end 158.223949 82.023949) (width 0.25) (layer "F.Cu") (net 19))
 (segment (start 155.683949 84.613949) (end 158.173949 84.613949) (width 0.25) (layer "F.Cu") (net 20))
 (segment (start 158.173949 84.613949) (end 158.223949 84.563949) (width 0.25) (layer "F.Cu") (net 20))
 (segment (start 158.173949 87.153949) (end 158.223949 87.103949) (width 0.25) (layer "F.Cu") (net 21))
 (segment (start 155.683949 87.153949) (end 158.173949 87.153949) (width 0.25) (layer "F.Cu") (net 21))
 (segment (start 158.173949 89.693949) (end 158.223949 89.643949) (width 0.25) (layer "F.Cu") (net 22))
 (segment (start 155.683949 89.693949) (end 158.173949 89.693949) (width 0.25) (layer "F.Cu") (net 22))
 (segment (start 155.683949 92.233949) (end 158.173949 92.233949) (width 0.25) (layer "F.Cu") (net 23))
 (segment (start 158.173949 92.233949) (end 158.223949 92.183949) (width 0.25) (layer "F.Cu") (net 23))
 (segment (start 158.173949 94.773949) (end 158.223949 94.723949) (width 0.25) (layer "F.Cu") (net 24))
 (segment (start 155.683949 94.773949) (end 158.173949 94.773949) (width 0.25) (layer "F.Cu") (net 24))
 (segment (start 155.683949 97.313949) (end 158.173949 97.313949) (width 0.25) (layer "F.Cu") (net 25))
 (segment (start 158.173949 97.313949) (end 158.223949 97.263949) (width 0.25) (layer "F.Cu") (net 25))
 (segment (start 152.926051 108.839) (end 151.511 107.423949) (width 0.25) (layer "F.Cu") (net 48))
 (segment (start 156.845 108.839) (end 152.926051 108.839) (width 0.25) (layer "F.Cu") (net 48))
 (via (at 156.845 108.839) (size 0.8) (drill 0.4) (layers "F.Cu" "B.Cu") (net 48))
 (segment (start 156.845 101.182898) (end 156.845 108.839) (width 0.25) (layer "B.Cu") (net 48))
 (segment (start 158.223949 99.803949) (end 156.845 101.182898) (width 0.25) (layer "B.Cu") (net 48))
 (segment (start 155.683949 102.393949) (end 158.173949 102.393949) (width 0.25) (layer "F.Cu") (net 27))
 (segment (start 158.173949 102.393949) (end 158.223949 102.343949) (width 0.25) (layer "F.Cu") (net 27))
 (segment (start 158.173949 104.933949) (end 158.223949 104.883949) (width 0.25) (layer "F.Cu") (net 10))
 (segment (start 155.683949 104.933949) (end 158.173949 104.933949) (width 0.25) (layer "F.Cu") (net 10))
 (segment (start 151.511 92.183949) (end 152.686 93.358949) (width 0.25) (layer "B.Cu") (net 10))
 (segment (start 152.686 101.936) (end 155.683949 104.933949) (width 0.25) (layer "B.Cu") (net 10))
 (segment (start 152.686 93.358949) (end 152.686 101.936) (width 0.25) (layer "B.Cu") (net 10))
 (segment (start 173.413949 107.473949) (end 173.463949 107.423949) (width 0.25) (layer "F.Cu") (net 29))
 (segment (start 170.923949 107.473949) (end 173.413949 107.473949) (width 0.25) (layer "F.Cu") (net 29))
 (segment (start 173.413949 104.933949) (end 173.463949 104.883949) (width 0.25) (layer "F.Cu") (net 30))
 (segment (start 170.923949 104.933949) (end 173.413949 104.933949) (width 0.25) (layer "F.Cu") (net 30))
 (segment (start 170.923949 102.393949) (end 173.413949 102.393949) (width 0.25) (layer "F.Cu") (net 31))
 (segment (start 173.413949 102.393949) (end 173.463949 102.343949) (width 0.25) (layer "F.Cu") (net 31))
 (segment (start 170.923949 99.853949) (end 173.413949 99.853949) (width 0.25) (layer "F.Cu") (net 32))
 (segment (start 173.413949 99.853949) (end 173.463949 99.803949) (width 0.25) (layer "F.Cu") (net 32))
 (segment (start 170.923949 94.773949) (end 173.413949 94.773949) (width 0.25) (layer "F.Cu") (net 34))
 (segment (start 173.413949 94.773949) (end 173.463949 94.723949) (width 0.25) (layer "F.Cu") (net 34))
 (segment (start 170.923949 92.233949) (end 173.413949 92.233949) (width 0.25) (layer "F.Cu") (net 35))
 (segment (start 173.413949 92.233949) (end 173.463949 92.183949) (width 0.25) (layer "F.Cu") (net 35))
 (segment (start 173.413949 89.693949) (end 173.463949 89.643949) (width 0.25) (layer "F.Cu") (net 36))
 (segment (start 170.923949 89.693949) (end 173.413949 89.693949) (width 0.25) (layer "F.Cu") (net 36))
 (segment (start 170.923949 87.153949) (end 173.413949 87.153949) (width 0.25) (layer "F.Cu") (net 37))
 (segment (start 173.413949 87.153949) (end 173.463949 87.103949) (width 0.25) (layer "F.Cu") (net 37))
 (segment (start 173.413949 84.613949) (end 173.463949 84.563949) (width 0.25) (layer "F.Cu") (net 38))
 (segment (start 170.923949 84.613949) (end 173.413949 84.613949) (width 0.25) (layer "F.Cu") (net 38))
 (segment (start 170.923949 82.073949) (end 173.413949 82.073949) (width 0.25) (layer "F.Cu") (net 39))
 (segment (start 173.413949 82.073949) (end 173.463949 82.023949) (width 0.25) (layer "F.Cu") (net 39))
 (segment (start 173.413949 79.533949) (end 173.463949 79.483949) (width 0.25) (layer "F.Cu") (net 40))
 (segment (start 170.923949 79.533949) (end 173.413949 79.533949) (width 0.25) (layer "F.Cu") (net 40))
 (segment (start 173.413949 76.993949) (end 173.463949 76.943949) (width 0.25) (layer "F.Cu") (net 41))
 (segment (start 170.923949 76.993949) (end 173.413949 76.993949) (width 0.25) (layer "F.Cu") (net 41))
 (segment (start 170.923949 74.453949) (end 173.413949 74.453949) (width 0.25) (layer "F.Cu") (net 42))
 (segment (start 173.413949 74.453949) (end 173.463949 74.403949) (width 0.25) (layer "F.Cu") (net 42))
 (segment (start 170.923949 71.913949) (end 173.413949 71.913949) (width 0.25) (layer "F.Cu") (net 43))
 (segment (start 173.413949 71.913949) (end 173.463949 71.863949) (width 0.25) (layer "F.Cu") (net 43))
 (segment (start 170.923949 69.373949) (end 173.413949 69.373949) (width 0.25) (layer "F.Cu") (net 44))
 (segment (start 173.413949 69.373949) (end 173.463949 69.323949) (width 0.25) (layer "F.Cu") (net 44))
 (segment (start 173.413949 66.833949) (end 173.463949 66.783949) (width 0.25) (layer "F.Cu") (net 45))
 (segment (start 170.923949 66.833949) (end 173.413949 66.833949) (width 0.25) (layer "F.Cu") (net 45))
 (segment (start 170.923949 64.293949) (end 173.413949 64.293949) (width 0.25) (layer "F.Cu") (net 46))
 (segment (start 173.413949 64.293949) (end 173.463949 64.243949) (width 0.25) (layer "F.Cu") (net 46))
 (segment (start 173.413949 61.753949) (end 173.463949 61.703949) (width 0.25) (layer "F.Cu") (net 47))
 (segment (start 170.923949 61.753949) (end 173.413949 61.753949) (width 0.25) (layer "F.Cu") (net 47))
 (segment (start 150.336 88.468949) (end 133.908051 88.468949) (width 0.25) (layer "F.Cu") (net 4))
 (segment (start 133.908051 88.468949) (end 133.858 88.519) (width 0.25) (layer "F.Cu") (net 4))
 (segment (start 151.511 89.643949) (end 150.336 88.468949) (width 0.25) (layer "F.Cu") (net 4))
 (via (at 133.858 88.519) (size 0.8) (drill 0.4) (layers "F.Cu" "B.Cu") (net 4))
 (segment (start 133.858 88.519) (end 133.858 98.053949) (width 0.25) (layer "B.Cu") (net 4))
 (segment (start 133.858 83.303949) (end 133.858 88.519) (width 0.25) (layer "B.Cu") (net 4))
 (segment (start 130.048 79.493949) (end 133.858 83.303949) (width 0.25) (layer "B.Cu") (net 4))
 (segment (start 154.382 106.172) (end 155.683949 107.473949) (width 0.25) (layer "F.Cu") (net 28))
 (segment (start 146.135051 99.228949) (end 146.138 99.226) (width 0.25) (layer "F.Cu") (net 28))
 (segment (start 146.177 106.172) (end 154.382 106.172) (width 0.25) (layer "F.Cu") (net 28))
 (segment (start 140.113 99.228949) (end 146.135051 99.228949) (width 0.25) (layer "F.Cu") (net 28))
 (segment (start 138.938 98.053949) (end 140.113 99.228949) (width 0.25) (layer "F.Cu") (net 28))
 (via (at 146.177 106.172) (size 0.8) (drill 0.4) (layers "F.Cu" "B.Cu") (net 28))
 (via (at 146.138 99.226) (size 0.8) (drill 0.4) (layers "F.Cu" "B.Cu") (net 28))
 (segment (start 146.138 106.133) (end 146.177 106.172) (width 0.25) (layer "B.Cu") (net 28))
 (segment (start 145.288 92.183949) (end 146.138 93.033949) (width 0.25) (layer "B.Cu") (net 28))
 (segment (start 146.138 93.033949) (end 146.138 106.133) (width 0.25) (layer "B.Cu") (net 28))
 (segment (start 146.463 83.198949) (end 168.288949 83.198949) (width 0.25) (layer "F.Cu") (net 33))
 (segment (start 168.288949 83.198949) (end 168.91 83.82) (width 0.25) (layer "F.Cu") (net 33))
 (segment (start 145.288 82.023949) (end 146.463 83.198949) (width 0.25) (layer "F.Cu") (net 33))
 (via (at 168.91 83.82) (size 0.8) (drill 0.4) (layers "F.Cu" "B.Cu") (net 33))
 (segment (start 141.478 85.833949) (end 145.288 82.023949) (width 0.25) (layer "B.Cu") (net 33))
 (segment (start 141.478 98.053949) (end 141.478 85.833949) (width 0.25) (layer "B.Cu") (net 33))
 (segment (start 168.91 95.3) (end 170.923949 97.313949) (width 0.25) (layer "B.Cu") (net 33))
 (segment (start 168.91 83.82) (end 168.91 95.3) (width 0.25) (layer "B.Cu") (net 33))
 (segment (start 163.231051 98.388949) (end 157.148949 98.388949) (width 0.25) (layer "F.Cu") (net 26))
 (segment (start 151.511 104.026898) (end 151.511 104.883949) (width 0.25) (layer "F.Cu") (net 26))
 (segment (start 157.148949 98.388949) (end 155.683949 99.853949) (width 0.25) (layer "F.Cu") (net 26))
 (segment (start 163.83 97.79) (end 163.231051 98.388949) (width 0.25) (layer "F.Cu") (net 26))
 (segment (start 155.683949 99.853949) (end 151.511 104.026898) (width 0.25) (layer "F.Cu") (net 26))
 (via (at 163.83 97.79) (size 0.8) (drill 0.4) (layers "F.Cu" "B.Cu") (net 26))
 (segment (start 170.923949 59.213949) (end 163.83 66.307898) (width 0.25) (layer "B.Cu") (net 26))
 (segment (start 163.83 66.307898) (end 163.83 97.79) (width 0.25) (layer "B.Cu") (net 26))
 (segment (start 140.843 103.613949) (end 144.653 103.613949) (width 0.25) (layer "F.Cu") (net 49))
 (segment (start 144.653 103.613949) (end 150.241 103.613949) (width 0.25) (layer "F.Cu") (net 49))
 (segment (start 150.241 103.613949) (end 151.511 102.343949) (width 0.25) (layer "F.Cu") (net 49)))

